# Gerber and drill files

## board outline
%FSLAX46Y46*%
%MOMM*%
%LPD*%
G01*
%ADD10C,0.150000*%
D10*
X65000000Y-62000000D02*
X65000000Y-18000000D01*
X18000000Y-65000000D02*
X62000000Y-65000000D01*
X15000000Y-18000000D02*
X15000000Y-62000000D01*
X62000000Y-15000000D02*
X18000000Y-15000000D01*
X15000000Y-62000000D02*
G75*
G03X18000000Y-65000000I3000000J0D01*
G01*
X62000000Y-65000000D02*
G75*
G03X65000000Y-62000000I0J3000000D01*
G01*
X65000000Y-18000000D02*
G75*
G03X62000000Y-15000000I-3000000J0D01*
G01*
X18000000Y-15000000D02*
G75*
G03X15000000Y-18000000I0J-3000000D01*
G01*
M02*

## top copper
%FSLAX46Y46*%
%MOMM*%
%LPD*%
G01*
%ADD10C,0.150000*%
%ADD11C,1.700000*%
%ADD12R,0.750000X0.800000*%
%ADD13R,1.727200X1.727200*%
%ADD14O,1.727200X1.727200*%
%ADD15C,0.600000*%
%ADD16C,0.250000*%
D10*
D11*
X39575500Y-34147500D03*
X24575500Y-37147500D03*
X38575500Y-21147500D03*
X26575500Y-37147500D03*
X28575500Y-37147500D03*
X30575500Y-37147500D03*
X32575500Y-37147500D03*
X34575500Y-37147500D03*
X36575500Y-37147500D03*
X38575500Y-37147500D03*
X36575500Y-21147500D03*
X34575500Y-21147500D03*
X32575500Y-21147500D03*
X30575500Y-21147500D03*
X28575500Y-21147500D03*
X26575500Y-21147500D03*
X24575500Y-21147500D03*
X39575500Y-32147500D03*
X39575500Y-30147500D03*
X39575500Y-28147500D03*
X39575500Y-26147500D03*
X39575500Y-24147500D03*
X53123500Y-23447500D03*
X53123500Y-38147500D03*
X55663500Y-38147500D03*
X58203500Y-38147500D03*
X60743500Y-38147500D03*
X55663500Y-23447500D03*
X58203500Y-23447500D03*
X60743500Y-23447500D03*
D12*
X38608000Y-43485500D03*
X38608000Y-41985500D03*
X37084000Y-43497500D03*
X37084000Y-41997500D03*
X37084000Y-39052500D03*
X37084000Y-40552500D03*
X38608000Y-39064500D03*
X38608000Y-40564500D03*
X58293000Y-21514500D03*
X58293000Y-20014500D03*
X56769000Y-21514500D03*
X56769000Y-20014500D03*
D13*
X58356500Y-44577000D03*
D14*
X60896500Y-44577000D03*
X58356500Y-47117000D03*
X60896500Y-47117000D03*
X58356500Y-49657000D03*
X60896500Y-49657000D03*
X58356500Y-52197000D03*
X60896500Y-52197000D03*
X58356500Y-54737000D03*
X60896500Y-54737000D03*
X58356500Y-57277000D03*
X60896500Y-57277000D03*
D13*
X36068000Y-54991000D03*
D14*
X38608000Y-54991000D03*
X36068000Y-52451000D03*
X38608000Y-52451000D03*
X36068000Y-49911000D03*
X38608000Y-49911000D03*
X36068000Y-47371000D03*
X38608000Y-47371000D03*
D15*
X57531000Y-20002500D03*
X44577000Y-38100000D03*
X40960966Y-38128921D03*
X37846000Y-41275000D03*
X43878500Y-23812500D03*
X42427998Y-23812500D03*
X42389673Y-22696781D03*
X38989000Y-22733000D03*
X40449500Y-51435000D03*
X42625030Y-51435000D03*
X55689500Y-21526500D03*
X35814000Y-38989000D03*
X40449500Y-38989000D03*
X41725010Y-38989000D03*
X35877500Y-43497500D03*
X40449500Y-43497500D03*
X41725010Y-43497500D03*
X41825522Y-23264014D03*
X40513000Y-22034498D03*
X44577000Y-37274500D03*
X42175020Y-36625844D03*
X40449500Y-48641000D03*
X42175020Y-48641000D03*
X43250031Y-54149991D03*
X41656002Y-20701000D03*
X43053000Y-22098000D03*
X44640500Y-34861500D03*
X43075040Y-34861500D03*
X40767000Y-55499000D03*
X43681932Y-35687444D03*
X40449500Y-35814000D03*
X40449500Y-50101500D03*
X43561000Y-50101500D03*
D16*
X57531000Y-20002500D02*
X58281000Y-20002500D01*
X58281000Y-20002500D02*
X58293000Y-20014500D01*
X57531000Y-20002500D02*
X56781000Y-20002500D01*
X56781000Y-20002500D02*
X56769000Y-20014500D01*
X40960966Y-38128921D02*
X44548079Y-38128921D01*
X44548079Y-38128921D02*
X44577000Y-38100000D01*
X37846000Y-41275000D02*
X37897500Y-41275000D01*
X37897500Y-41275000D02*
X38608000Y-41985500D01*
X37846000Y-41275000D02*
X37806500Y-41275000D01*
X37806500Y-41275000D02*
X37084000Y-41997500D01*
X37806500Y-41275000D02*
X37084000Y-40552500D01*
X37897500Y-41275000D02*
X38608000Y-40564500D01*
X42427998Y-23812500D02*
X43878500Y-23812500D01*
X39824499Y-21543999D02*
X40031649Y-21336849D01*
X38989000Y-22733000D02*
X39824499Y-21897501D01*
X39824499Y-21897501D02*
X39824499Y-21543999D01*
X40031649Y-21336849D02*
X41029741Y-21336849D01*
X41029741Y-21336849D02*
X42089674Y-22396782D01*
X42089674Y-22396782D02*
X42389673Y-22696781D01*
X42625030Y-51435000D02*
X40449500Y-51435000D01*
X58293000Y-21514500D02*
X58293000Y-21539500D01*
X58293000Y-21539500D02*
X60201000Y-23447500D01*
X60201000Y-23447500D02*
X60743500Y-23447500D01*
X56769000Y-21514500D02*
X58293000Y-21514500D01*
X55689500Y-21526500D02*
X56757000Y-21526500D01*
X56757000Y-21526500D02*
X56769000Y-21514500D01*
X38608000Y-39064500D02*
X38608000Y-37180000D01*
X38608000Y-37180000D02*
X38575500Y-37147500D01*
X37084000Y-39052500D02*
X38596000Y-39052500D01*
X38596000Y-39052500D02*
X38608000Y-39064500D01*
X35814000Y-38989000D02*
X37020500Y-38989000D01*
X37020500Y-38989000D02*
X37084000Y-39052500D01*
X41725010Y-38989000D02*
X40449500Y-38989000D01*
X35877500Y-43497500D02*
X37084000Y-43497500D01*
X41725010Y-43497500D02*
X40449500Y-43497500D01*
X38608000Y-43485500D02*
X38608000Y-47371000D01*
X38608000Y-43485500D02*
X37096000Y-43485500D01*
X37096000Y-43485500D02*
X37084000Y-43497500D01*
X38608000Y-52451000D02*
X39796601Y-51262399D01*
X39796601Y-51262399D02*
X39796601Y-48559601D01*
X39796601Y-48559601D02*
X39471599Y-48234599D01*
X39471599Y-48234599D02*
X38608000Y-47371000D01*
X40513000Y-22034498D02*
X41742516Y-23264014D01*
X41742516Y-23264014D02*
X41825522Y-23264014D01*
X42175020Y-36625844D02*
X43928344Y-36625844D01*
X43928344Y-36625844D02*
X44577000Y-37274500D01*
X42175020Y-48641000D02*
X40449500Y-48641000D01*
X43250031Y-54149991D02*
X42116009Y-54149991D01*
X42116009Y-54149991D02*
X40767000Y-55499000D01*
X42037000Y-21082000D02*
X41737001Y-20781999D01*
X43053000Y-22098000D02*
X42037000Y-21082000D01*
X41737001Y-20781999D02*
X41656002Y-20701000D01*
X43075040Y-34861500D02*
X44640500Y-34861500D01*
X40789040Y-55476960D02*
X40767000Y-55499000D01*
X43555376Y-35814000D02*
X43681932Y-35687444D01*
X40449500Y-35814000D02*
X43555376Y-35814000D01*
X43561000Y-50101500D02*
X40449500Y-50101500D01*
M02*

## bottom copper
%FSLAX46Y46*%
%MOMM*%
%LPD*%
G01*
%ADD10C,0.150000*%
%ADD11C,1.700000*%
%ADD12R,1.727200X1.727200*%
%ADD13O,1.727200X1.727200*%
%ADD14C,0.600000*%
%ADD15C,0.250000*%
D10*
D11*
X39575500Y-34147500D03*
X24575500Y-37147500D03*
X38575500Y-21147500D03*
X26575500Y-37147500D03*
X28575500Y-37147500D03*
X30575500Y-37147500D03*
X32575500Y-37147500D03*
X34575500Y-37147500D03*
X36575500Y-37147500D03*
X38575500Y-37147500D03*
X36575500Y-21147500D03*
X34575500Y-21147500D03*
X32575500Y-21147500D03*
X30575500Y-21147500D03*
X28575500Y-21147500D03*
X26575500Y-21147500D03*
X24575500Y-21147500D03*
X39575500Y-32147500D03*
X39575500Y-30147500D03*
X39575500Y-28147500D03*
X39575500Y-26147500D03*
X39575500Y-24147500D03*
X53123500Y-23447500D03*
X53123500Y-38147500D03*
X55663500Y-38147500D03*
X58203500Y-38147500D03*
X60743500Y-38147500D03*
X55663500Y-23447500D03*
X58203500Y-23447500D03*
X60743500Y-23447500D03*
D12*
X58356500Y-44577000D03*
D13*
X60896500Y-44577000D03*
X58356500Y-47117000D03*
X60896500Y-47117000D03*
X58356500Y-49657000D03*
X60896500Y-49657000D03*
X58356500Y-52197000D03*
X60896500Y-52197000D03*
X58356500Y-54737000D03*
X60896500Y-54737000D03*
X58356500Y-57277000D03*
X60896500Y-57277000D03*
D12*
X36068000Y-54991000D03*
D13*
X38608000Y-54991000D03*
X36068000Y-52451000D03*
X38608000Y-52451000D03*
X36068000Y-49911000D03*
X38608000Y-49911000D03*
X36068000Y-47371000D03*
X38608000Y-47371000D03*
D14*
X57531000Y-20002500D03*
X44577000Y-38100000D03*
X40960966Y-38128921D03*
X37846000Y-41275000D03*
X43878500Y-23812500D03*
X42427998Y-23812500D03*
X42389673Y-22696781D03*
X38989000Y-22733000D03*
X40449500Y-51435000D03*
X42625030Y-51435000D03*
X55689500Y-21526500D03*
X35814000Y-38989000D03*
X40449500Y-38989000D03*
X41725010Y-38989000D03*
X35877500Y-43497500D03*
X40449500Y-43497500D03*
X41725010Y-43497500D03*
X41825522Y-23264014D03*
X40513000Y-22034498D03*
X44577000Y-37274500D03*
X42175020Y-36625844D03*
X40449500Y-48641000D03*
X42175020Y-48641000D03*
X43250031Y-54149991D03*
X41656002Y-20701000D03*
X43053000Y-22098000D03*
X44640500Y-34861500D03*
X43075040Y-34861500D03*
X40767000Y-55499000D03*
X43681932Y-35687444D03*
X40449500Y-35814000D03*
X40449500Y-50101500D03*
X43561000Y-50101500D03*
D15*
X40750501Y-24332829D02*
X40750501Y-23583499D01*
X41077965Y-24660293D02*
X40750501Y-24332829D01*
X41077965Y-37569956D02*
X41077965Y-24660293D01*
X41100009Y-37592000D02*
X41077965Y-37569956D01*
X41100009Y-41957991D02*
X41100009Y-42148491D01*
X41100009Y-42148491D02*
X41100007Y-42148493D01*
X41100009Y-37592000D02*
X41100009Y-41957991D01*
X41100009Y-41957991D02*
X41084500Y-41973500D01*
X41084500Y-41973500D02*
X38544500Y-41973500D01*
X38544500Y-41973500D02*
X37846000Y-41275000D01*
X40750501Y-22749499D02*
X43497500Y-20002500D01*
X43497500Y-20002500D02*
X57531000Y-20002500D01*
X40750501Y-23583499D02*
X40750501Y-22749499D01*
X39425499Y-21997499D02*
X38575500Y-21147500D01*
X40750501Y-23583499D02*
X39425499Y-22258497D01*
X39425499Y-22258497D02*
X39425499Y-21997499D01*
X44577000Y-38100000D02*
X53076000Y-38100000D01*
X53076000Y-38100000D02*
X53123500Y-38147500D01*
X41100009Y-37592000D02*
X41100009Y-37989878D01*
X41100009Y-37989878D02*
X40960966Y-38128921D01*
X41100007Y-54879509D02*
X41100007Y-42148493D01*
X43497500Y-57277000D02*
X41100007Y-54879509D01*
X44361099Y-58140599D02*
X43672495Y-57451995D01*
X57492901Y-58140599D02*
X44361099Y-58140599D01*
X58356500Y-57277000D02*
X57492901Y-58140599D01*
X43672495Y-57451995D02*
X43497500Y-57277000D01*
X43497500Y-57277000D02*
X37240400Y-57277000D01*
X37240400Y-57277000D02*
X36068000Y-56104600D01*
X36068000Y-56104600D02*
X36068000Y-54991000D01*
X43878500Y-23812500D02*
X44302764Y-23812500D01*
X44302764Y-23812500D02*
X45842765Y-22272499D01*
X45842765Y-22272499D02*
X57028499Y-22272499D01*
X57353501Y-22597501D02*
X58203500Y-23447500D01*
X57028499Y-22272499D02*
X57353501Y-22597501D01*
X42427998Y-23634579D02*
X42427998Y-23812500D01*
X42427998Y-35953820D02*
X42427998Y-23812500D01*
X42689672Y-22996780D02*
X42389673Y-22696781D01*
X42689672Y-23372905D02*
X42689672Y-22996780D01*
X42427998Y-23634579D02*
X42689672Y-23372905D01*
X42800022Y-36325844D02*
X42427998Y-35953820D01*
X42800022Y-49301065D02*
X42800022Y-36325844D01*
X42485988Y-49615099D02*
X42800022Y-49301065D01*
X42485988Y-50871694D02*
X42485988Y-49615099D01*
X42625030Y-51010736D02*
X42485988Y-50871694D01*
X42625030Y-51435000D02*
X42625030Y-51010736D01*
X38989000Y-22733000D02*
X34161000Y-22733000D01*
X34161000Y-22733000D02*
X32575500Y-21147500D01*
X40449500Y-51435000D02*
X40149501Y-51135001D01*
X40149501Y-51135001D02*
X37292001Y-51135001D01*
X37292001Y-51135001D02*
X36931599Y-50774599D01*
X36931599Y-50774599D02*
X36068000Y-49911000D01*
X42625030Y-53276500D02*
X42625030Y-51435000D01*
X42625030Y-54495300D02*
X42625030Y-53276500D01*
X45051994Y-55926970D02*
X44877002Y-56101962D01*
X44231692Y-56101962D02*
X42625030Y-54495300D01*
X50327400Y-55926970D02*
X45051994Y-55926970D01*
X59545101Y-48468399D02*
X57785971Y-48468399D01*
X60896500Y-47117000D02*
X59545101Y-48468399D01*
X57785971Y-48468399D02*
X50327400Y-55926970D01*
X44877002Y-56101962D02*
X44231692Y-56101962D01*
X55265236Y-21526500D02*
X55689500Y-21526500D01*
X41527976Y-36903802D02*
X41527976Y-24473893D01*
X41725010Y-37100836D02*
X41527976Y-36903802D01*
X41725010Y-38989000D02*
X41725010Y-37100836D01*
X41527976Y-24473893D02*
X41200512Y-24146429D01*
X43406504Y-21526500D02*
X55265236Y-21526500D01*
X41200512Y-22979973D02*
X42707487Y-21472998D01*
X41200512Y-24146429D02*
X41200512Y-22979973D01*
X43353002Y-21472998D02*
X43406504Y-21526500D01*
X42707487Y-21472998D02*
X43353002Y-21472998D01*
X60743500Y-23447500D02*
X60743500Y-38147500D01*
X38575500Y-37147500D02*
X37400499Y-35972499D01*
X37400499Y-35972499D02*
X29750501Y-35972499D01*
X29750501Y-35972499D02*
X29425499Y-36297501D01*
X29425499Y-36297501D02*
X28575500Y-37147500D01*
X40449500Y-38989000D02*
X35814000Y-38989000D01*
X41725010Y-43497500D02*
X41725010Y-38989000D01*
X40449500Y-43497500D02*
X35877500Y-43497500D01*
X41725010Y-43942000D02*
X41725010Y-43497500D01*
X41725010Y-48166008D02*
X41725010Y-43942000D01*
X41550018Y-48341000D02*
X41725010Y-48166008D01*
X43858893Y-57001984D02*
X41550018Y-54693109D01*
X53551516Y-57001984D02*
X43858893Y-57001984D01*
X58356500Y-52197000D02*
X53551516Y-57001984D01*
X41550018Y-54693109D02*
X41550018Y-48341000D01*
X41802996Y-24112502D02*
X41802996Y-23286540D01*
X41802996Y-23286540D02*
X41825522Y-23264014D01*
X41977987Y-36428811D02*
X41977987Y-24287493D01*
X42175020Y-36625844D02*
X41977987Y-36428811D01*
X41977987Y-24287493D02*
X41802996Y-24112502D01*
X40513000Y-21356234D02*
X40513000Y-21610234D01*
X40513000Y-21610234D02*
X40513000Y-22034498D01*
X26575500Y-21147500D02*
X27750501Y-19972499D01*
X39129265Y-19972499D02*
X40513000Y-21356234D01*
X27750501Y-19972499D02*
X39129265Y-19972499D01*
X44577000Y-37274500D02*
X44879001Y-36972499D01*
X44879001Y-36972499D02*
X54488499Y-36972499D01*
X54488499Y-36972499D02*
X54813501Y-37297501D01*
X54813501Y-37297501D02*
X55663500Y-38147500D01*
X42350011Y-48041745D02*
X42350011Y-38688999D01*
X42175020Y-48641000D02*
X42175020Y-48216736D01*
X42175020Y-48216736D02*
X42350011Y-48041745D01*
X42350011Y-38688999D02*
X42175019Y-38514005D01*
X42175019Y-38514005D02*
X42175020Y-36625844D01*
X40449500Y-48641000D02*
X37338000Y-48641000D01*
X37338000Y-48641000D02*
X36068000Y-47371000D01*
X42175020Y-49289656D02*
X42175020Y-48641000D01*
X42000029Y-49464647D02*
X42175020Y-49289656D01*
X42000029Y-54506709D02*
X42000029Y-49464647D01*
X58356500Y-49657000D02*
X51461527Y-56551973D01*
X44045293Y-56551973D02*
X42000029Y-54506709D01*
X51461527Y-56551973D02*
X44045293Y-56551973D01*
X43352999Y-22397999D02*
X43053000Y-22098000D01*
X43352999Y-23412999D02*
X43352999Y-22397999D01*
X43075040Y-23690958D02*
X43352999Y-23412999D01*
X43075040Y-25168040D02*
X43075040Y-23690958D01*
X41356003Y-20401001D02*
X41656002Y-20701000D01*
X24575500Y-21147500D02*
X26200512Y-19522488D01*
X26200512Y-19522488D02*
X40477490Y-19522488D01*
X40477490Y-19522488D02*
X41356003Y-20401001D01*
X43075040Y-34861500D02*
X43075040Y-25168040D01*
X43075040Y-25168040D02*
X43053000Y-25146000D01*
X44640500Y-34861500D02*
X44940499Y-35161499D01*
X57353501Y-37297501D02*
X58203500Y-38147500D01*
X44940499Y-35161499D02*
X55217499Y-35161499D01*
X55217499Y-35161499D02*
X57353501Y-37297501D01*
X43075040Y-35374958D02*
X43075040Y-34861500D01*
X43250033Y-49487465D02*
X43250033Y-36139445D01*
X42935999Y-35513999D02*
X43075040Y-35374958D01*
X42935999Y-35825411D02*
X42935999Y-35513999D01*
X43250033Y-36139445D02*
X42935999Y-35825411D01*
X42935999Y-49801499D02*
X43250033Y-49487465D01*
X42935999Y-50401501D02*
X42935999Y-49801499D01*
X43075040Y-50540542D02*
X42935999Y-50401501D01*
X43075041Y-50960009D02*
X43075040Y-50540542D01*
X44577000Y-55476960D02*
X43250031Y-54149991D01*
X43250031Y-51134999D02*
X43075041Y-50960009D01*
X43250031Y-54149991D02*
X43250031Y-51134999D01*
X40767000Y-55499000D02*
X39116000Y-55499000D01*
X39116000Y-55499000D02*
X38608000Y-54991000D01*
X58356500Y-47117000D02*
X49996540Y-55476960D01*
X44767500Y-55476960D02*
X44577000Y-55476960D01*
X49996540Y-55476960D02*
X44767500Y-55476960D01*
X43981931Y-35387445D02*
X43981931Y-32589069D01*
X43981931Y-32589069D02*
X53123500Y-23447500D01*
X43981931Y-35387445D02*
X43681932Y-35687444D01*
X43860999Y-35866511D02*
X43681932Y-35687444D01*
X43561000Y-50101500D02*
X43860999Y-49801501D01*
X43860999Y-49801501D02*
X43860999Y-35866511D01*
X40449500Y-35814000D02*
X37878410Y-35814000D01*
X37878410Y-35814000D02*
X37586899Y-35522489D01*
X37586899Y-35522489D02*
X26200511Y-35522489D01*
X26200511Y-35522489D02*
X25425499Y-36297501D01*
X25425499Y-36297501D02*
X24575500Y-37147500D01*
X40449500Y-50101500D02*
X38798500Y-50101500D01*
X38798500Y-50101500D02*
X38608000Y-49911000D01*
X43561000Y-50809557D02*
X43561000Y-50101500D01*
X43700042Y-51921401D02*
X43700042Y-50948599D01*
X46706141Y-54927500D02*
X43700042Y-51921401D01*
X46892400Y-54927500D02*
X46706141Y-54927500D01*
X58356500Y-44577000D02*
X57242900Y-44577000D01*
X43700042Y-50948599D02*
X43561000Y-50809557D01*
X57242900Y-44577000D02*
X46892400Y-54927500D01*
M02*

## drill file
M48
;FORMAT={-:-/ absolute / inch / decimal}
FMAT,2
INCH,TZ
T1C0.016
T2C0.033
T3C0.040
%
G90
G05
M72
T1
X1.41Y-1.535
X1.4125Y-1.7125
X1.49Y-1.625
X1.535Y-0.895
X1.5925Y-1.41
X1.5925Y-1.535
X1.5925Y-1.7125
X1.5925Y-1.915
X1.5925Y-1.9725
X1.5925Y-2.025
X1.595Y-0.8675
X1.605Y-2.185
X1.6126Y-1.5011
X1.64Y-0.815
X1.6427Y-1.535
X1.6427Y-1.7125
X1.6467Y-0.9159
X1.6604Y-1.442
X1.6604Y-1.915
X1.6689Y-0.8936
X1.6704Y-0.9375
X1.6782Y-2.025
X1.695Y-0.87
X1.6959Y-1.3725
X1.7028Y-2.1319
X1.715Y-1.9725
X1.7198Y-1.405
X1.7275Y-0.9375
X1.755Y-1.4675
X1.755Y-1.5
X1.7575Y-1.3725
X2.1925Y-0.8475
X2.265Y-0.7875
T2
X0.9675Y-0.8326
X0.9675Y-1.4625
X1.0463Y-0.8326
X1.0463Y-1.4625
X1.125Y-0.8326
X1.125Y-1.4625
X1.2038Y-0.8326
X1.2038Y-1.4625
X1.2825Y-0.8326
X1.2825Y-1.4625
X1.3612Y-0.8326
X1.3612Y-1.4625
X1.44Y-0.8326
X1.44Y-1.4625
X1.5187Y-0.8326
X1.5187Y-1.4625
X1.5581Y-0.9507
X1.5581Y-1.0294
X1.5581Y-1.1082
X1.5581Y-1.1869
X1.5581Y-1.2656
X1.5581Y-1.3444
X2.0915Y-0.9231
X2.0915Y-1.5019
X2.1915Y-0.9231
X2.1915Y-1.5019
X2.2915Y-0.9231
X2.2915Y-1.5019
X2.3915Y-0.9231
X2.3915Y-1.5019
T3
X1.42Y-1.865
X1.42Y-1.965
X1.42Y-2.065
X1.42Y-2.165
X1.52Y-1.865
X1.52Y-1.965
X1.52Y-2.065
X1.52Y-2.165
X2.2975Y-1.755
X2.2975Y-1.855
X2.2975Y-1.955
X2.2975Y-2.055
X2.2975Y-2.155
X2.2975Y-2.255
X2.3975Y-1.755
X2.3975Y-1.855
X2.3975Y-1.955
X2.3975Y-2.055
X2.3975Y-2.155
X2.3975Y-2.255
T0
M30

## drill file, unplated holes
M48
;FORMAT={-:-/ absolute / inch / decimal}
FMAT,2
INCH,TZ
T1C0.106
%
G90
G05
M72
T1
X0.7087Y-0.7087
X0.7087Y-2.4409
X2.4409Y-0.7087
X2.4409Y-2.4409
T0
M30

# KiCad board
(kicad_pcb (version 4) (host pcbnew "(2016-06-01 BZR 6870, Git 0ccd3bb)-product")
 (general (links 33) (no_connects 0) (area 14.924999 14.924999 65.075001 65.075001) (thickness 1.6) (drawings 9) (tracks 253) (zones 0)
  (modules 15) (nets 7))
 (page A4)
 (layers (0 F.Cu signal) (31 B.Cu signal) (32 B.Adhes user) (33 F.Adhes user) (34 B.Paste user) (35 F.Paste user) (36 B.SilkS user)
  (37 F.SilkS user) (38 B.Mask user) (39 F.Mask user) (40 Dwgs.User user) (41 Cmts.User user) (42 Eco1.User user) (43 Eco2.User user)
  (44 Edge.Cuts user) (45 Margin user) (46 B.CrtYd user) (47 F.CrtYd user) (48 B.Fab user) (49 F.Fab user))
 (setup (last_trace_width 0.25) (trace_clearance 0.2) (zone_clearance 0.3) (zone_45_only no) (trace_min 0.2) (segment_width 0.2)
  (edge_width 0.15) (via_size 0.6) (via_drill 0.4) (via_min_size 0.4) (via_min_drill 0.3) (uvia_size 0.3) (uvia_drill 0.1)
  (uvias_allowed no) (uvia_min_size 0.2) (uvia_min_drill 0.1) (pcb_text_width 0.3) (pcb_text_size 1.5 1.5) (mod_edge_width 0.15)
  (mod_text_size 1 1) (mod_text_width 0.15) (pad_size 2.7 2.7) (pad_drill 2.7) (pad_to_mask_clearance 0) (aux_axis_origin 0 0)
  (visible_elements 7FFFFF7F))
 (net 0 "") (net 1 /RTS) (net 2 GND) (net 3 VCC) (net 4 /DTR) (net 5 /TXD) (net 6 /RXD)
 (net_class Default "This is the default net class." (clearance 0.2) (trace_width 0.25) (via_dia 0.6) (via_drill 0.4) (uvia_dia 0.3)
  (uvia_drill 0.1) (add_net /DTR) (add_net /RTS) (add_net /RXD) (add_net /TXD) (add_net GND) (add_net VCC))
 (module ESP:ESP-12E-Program (layer F.Cu) (at 27.5755 29.1475 90)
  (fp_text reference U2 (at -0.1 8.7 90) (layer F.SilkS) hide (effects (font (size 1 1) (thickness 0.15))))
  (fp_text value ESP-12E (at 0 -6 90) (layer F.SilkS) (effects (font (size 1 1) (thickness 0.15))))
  (pad 9 thru_hole circle (at -5 12 90) (size 1.7 1.7) (drill 0.85) (layers *.Cu *.Mask F.SilkS))
  (pad 1 thru_hole circle (at -8 -3 90) (size 1.7 1.7) (drill 0.85) (layers *.Cu *.Mask F.SilkS) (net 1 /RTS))
  (pad 15 thru_hole circle (at 8 11 90) (size 1.7 1.7) (drill 0.85) (layers *.Cu *.Mask F.SilkS) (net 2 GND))
  (pad 2 thru_hole circle (at -8 -1 90) (size 1.7 1.7) (drill 0.85) (layers *.Cu *.Mask F.SilkS))
  (pad 3 thru_hole circle (at -8 1 90) (size 1.7 1.7) (drill 0.85) (layers *.Cu *.Mask F.SilkS) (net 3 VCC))
  (pad 4 thru_hole circle (at -8 3 90) (size 1.7 1.7) (drill 0.85) (layers *.Cu *.Mask F.SilkS))
  (pad 5 thru_hole circle (at -8 5 90) (size 1.7 1.7) (drill 0.85) (layers *.Cu *.Mask F.SilkS))
  (pad 6 thru_hole circle (at -8 7 90) (size 1.7 1.7) (drill 0.85) (layers *.Cu *.Mask F.SilkS))
  (pad 7 thru_hole circle (at -8 9 90) (size 1.7 1.7) (drill 0.85) (layers *.Cu *.Mask F.SilkS))
  (pad 8 thru_hole circle (at -8 11 90) (size 1.7 1.7) (drill 0.85) (layers *.Cu *.Mask F.SilkS) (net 3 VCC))
  (pad 16 thru_hole circle (at 8 9 90) (size 1.7 1.7) (drill 0.85) (layers *.Cu *.Mask F.SilkS))
  (pad 17 thru_hole circle (at 8 7 90) (size 1.7 1.7) (drill 0.85) (layers *.Cu *.Mask F.SilkS))
  (pad 18 thru_hole circle (at 8 5 90) (size 1.7 1.7) (drill 0.85) (layers *.Cu *.Mask F.SilkS) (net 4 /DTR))
  (pad 19 thru_hole circle (at 8 3 90) (size 1.7 1.7) (drill 0.85) (layers *.Cu *.Mask F.SilkS))
  (pad 20 thru_hole circle (at 8 1 90) (size 1.7 1.7) (drill 0.85) (layers *.Cu *.Mask F.SilkS))
  (pad 21 thru_hole circle (at 8 -1 90) (size 1.7 1.7) (drill 0.85) (layers *.Cu *.Mask F.SilkS) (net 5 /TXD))
  (pad 22 thru_hole circle (at 8 -3 90) (size 1.7 1.7) (drill 0.85) (layers *.Cu *.Mask F.SilkS) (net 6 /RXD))
  (pad 10 thru_hole circle (at -3 12 90) (size 1.7 1.7) (drill 0.85) (layers *.Cu *.Mask F.SilkS))
  (pad 11 thru_hole circle (at -1 12 90) (size 1.7 1.7) (drill 0.85) (layers *.Cu *.Mask F.SilkS))
  (pad 12 thru_hole circle (at 1 12 90) (size 1.7 1.7) (drill 0.85) (layers *.Cu *.Mask F.SilkS))
  (pad 13 thru_hole circle (at 3 12 90) (size 1.7 1.7) (drill 0.85) (layers *.Cu *.Mask F.SilkS))
  (pad 14 thru_hole circle (at 5 12 90) (size 1.7 1.7) (drill 0.85) (layers *.Cu *.Mask F.SilkS)))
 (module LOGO (layer F.Cu) (at 49.022 53.467 90)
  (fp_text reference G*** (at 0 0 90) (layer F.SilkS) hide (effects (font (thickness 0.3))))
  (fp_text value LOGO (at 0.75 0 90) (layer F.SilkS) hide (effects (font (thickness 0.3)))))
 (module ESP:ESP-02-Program (layer F.Cu) (at 54.6735 30.7975 90)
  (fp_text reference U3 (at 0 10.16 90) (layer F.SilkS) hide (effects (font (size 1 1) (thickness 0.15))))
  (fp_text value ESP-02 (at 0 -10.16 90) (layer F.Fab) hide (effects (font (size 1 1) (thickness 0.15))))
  (pad 8 thru_hole circle (at 7.35 -1.55 90) (size 1.7 1.7) (drill 0.85) (layers *.Cu *.Mask F.SilkS) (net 1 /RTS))
  (pad 1 thru_hole circle (at -7.35 -1.55 90) (size 1.7 1.7) (drill 0.85) (layers *.Cu *.Mask F.SilkS) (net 2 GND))
  (pad 2 thru_hole circle (at -7.35 0.99 90) (size 1.7 1.7) (drill 0.85) (layers *.Cu *.Mask F.SilkS) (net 5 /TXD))
  (pad 3 thru_hole circle (at -7.35 3.53 90) (size 1.7 1.7) (drill 0.85) (layers *.Cu *.Mask F.SilkS) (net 6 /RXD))
  (pad 4 thru_hole circle (at -7.35 6.07 90) (size 1.7 1.7) (drill 0.85) (layers *.Cu *.Mask F.SilkS) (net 3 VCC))
  (pad 7 thru_hole circle (at 7.35 0.99 90) (size 1.7 1.7) (drill 0.85) (layers *.Cu *.Mask F.SilkS))
  (pad 6 thru_hole circle (at 7.35 3.53 90) (size 1.7 1.7) (drill 0.85) (layers *.Cu *.Mask F.SilkS) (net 4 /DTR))
  (pad 5 thru_hole circle (at 7.35 6.07 90) (size 1.7 1.7) (drill 0.85) (layers *.Cu *.Mask F.SilkS) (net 3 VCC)))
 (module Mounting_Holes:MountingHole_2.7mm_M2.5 (layer F.Cu) (at 18 18)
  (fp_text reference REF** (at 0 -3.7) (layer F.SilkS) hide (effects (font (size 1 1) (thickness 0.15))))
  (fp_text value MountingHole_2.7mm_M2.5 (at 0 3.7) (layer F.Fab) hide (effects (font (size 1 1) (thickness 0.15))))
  (pad "" np_thru_hole circle (at 0 0) (size 2.7 2.7) (drill 2.7) (layers *.Cu *.Mask F.SilkS)))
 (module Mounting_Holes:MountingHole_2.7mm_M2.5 (layer F.Cu) (at 18 62)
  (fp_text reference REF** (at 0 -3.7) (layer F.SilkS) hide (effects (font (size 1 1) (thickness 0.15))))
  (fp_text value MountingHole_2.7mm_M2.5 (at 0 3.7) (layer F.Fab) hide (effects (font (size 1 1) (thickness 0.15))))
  (pad 1 np_thru_hole circle (at 0 0) (size 2.7 2.7) (drill 2.7) (layers *.Cu *.Mask F.SilkS)))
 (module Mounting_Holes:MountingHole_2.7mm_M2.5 (layer F.Cu) (at 62 62)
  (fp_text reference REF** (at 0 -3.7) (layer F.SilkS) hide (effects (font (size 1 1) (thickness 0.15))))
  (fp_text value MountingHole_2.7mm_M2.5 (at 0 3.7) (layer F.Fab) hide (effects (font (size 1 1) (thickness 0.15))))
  (pad 1 np_thru_hole circle (at 0 0) (size 2.7 2.7) (drill 2.7) (layers *.Cu *.Mask F.SilkS)))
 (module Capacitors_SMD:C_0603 (layer F.Cu) (at 38.608 42.7355 90)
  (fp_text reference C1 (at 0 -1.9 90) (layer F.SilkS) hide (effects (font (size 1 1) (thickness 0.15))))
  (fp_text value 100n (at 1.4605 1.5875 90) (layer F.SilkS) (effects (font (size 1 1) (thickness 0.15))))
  (pad 1 smd rect (at -0.75 0 90) (size 0.8 0.75) (layers F.Cu F.Paste F.Mask) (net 3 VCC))
  (pad 2 smd rect (at 0.75 0 90) (size 0.8 0.75) (layers F.Cu F.Paste F.Mask) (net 2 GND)))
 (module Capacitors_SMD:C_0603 (layer F.Cu) (at 37.084 42.7475 90)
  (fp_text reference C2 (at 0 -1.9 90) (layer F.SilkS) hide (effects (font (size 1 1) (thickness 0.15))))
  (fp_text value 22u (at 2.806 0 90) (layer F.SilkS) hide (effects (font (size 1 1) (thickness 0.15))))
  (pad 1 smd rect (at -0.75 0 90) (size 0.8 0.75) (layers F.Cu F.Paste F.Mask) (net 3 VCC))
  (pad 2 smd rect (at 0.75 0 90) (size 0.8 0.75) (layers F.Cu F.Paste F.Mask) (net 2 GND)))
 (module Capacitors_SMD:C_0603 (layer F.Cu) (at 37.084 39.8025 270)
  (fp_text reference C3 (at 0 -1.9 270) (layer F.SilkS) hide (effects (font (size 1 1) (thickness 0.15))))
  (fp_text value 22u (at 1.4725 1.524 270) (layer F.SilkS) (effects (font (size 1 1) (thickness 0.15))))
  (pad 1 smd rect (at -0.75 0 270) (size 0.8 0.75) (layers F.Cu F.Paste F.Mask) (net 3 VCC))
  (pad 2 smd rect (at 0.75 0 270) (size 0.8 0.75) (layers F.Cu F.Paste F.Mask) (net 2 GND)))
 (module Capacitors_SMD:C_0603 (layer F.Cu) (at 38.608 39.8145 270)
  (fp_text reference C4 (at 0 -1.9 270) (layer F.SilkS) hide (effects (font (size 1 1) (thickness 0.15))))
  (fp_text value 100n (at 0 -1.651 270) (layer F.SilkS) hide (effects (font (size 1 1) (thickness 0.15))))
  (pad 1 smd rect (at -0.75 0 270) (size 0.8 0.75) (layers F.Cu F.Paste F.Mask) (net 3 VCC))
  (pad 2 smd rect (at 0.75 0 270) (size 0.8 0.75) (layers F.Cu F.Paste F.Mask) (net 2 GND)))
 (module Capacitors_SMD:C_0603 (layer F.Cu) (at 58.293 20.7645 90)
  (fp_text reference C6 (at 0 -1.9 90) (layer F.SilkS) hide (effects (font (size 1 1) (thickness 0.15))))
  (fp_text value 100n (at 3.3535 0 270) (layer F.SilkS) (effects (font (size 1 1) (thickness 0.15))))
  (pad 1 smd rect (at -0.75 0 90) (size 0.8 0.75) (layers F.Cu F.Paste F.Mask) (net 3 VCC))
  (pad 2 smd rect (at 0.75 0 90) (size 0.8 0.75) (layers F.Cu F.Paste F.Mask) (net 2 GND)))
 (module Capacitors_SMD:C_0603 (layer F.Cu) (at 56.769 20.7645 90)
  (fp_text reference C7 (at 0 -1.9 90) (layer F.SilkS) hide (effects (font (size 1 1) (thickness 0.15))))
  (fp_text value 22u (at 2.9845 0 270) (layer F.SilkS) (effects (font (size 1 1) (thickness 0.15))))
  (pad 1 smd rect (at -0.75 0 90) (size 0.8 0.75) (layers F.Cu F.Paste F.Mask) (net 3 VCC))
  (pad 2 smd rect (at 0.75 0 90) (size 0.8 0.75) (layers F.Cu F.Paste F.Mask) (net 2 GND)))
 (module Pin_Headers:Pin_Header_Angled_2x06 (layer F.Cu) (at 58.3565 44.577)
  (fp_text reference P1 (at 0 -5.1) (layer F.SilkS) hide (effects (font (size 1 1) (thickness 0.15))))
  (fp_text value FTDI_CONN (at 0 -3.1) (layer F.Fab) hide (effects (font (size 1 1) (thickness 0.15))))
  (pad 1 thru_hole rect (at 0 0) (size 1.7272 1.7272) (drill 1.016) (layers *.Cu *.Mask F.SilkS) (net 1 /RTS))
  (pad 2 thru_hole oval (at 2.54 0) (size 1.7272 1.7272) (drill 1.016) (layers *.Cu *.Mask F.SilkS))
  (pad 3 thru_hole oval (at 0 2.54) (size 1.7272 1.7272) (drill 1.016) (layers *.Cu *.Mask F.SilkS) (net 6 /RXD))
  (pad 4 thru_hole oval (at 2.54 2.54) (size 1.7272 1.7272) (drill 1.016) (layers *.Cu *.Mask F.SilkS) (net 4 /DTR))
  (pad 5 thru_hole oval (at 0 5.08) (size 1.7272 1.7272) (drill 1.016) (layers *.Cu *.Mask F.SilkS) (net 5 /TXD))
  (pad 6 thru_hole oval (at 2.54 5.08) (size 1.7272 1.7272) (drill 1.016) (layers *.Cu *.Mask F.SilkS))
  (pad 7 thru_hole oval (at 0 7.62) (size 1.7272 1.7272) (drill 1.016) (layers *.Cu *.Mask F.SilkS) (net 3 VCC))
  (pad 8 thru_hole oval (at 2.54 7.62) (size 1.7272 1.7272) (drill 1.016) (layers *.Cu *.Mask F.SilkS))
  (pad 9 thru_hole oval (at 0 10.16) (size 1.7272 1.7272) (drill 1.016) (layers *.Cu *.Mask F.SilkS))
  (pad 10 thru_hole oval (at 2.54 10.16) (size 1.7272 1.7272) (drill 1.016) (layers *.Cu *.Mask F.SilkS))
  (pad 11 thru_hole oval (at 0 12.7) (size 1.7272 1.7272) (drill 1.016) (layers *.Cu *.Mask F.SilkS) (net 2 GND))
  (pad 12 thru_hole oval (at 2.54 12.7) (size 1.7272 1.7272) (drill 1.016) (layers *.Cu *.Mask F.SilkS)))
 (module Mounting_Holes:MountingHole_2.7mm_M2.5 (layer F.Cu) (at 62 18)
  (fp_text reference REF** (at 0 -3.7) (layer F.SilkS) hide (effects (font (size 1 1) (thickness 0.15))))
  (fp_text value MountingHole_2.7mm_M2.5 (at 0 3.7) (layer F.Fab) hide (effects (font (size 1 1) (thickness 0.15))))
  (pad 1 np_thru_hole circle (at 0 0) (size 2.7 2.7) (drill 2.7) (layers *.Cu *.Mask F.SilkS)))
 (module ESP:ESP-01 (layer F.Cu) (at 37.338 51.181 90)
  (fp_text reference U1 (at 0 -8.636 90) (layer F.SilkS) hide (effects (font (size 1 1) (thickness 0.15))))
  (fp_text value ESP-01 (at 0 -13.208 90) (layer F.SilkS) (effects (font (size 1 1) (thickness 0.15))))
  (pad 1 thru_hole rect (at -3.81 -1.27 90) (size 1.7272 1.7272) (drill 1.016) (layers *.Cu *.Mask F.SilkS) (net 2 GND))
  (pad 2 thru_hole oval (at -3.81 1.27 90) (size 1.7272 1.7272) (drill 1.016) (layers *.Cu *.Mask F.SilkS) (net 6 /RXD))
  (pad 3 thru_hole oval (at -1.27 -1.27 90) (size 1.7272 1.7272) (drill 1.016) (layers *.Cu *.Mask F.SilkS))
  (pad 4 thru_hole oval (at -1.27 1.27 90) (size 1.7272 1.7272) (drill 1.016) (layers *.Cu *.Mask F.SilkS) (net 3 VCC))
  (pad 5 thru_hole oval (at 1.27 -1.27 90) (size 1.7272 1.7272) (drill 1.016) (layers *.Cu *.Mask F.SilkS) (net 4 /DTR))
  (pad 6 thru_hole oval (at 1.27 1.27 90) (size 1.7272 1.7272) (drill 1.016) (layers *.Cu *.Mask F.SilkS) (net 1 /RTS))
  (pad 7 thru_hole oval (at 3.81 -1.27 90) (size 1.7272 1.7272) (drill 1.016) (layers *.Cu *.Mask F.SilkS) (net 5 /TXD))
  (pad 8 thru_hole oval (at 3.81 1.27 90) (size 1.7272 1.7272) (drill 1.016) (layers *.Cu *.Mask F.SilkS) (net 3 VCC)))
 (gr_line (start 65 62) (end 65 18) (layer Edge.Cuts) (width 0.15))
 (gr_line (start 18 65) (end 62 65) (layer Edge.Cuts) (width 0.15))
 (gr_line (start 15 18) (end 15 62) (layer Edge.Cuts) (width 0.15))
 (gr_line (start 62 15) (end 18 15) (layer Edge.Cuts) (width 0.15))
 (gr_arc (start 18 62) (end 18 65) (angle 90) (layer Edge.Cuts) (width 0.15))
 (gr_arc (start 62 62) (end 65 62) (angle 90) (layer Edge.Cuts) (width 0.15))
 (gr_arc (start 62 18) (end 62 15) (angle 90) (layer Edge.Cuts) (width 0.15))
 (gr_arc (start 18 18) (end 15 18) (angle 90) (layer Edge.Cuts) (width 0.15))
 (segment (start 40.750501 24.332829) (end 40.750501 23.583499) (width 0.25) (layer B.Cu) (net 2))
 (segment (start 41.077965 24.660293) (end 40.750501 24.332829) (width 0.25) (layer B.Cu) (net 2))
 (segment (start 41.077965 37.569956) (end 41.077965 24.660293) (width 0.25) (layer B.Cu) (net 2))
 (segment (start 41.100009 37.592) (end 41.077965 37.569956) (width 0.25) (layer B.Cu) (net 2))
 (segment (start 41.100009 41.957991) (end 41.100009 42.148491) (width 0.25) (layer B.Cu) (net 2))
 (segment (start 41.100009 42.148491) (end 41.100007 42.148493) (width 0.25) (layer B.Cu) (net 2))
 (segment (start 41.100009 37.592) (end 41.100009 41.957991) (width 0.25) (layer B.Cu) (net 2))
 (segment (start 41.100009 41.957991) (end 41.0845 41.9735) (width 0.25) (layer B.Cu) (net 2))
 (segment (start 41.0845 41.9735) (end 38.5445 41.9735) (width 0.25) (layer B.Cu) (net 2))
 (segment (start 38.5445 41.9735) (end 37.846 41.275) (width 0.25) (layer B.Cu) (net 2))
 (segment (start 57.531 20.0025) (end 58.281 20.0025) (width 0.25) (layer F.Cu) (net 2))
 (segment (start 58.281 20.0025) (end 58.293 20.0145) (width 0.25) (layer F.Cu) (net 2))
 (segment (start 57.531 20.0025) (end 56.781 20.0025) (width 0.25) (layer F.Cu) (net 2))
 (segment (start 56.781 20.0025) (end 56.769 20.0145) (width 0.25) (layer F.Cu) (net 2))
 (segment (start 40.750501 22.749499) (end 43.4975 20.0025) (width 0.25) (layer B.Cu) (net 2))
 (segment (start 43.4975 20.0025) (end 57.531 20.0025) (width 0.25) (layer B.Cu) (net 2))
 (via (at 57.531 20.0025) (size 0.6) (drill 0.4) (layers F.Cu B.Cu) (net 2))
 (segment (start 40.750501 23.583499) (end 40.750501 22.749499) (width 0.25) (layer B.Cu) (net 2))
 (segment (start 39.425499 21.997499) (end 38.5755 21.1475) (width 0.25) (layer B.Cu) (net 2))
 (segment (start 40.750501 23.583499) (end 39.425499 22.258497) (width 0.25) (layer B.Cu) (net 2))
 (segment (start 39.425499 22.258497) (end 39.425499 21.997499) (width 0.25) (layer B.Cu) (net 2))
 (segment (start 44.577 38.1) (end 53.076 38.1) (width 0.25) (layer B.Cu) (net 2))
 (segment (start 53.076 38.1) (end 53.1235 38.1475) (width 0.25) (layer B.Cu) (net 2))
 (segment (start 40.960966 38.128921) (end 44.548079 38.128921) (width 0.25) (layer F.Cu) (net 2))
 (segment (start 44.548079 38.128921) (end 44.577 38.1) (width 0.25) (layer F.Cu) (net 2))
 (via (at 44.577 38.1) (size 0.6) (drill 0.4) (layers F.Cu B.Cu) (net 2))
 (segment (start 41.100009 37.592) (end 41.100009 37.989878) (width 0.25) (layer B.Cu) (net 2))
 (segment (start 41.100009 37.989878) (end 40.960966 38.128921) (width 0.25) (layer B.Cu) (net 2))
 (via (at 40.960966 38.128921) (size 0.6) (drill 0.4) (layers F.Cu B.Cu) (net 2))
 (segment (start 41.100007 54.879509) (end 41.100007 42.148493) (width 0.25) (layer B.Cu) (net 2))
 (segment (start 43.4975 57.277) (end 41.100007 54.879509) (width 0.25) (layer B.Cu) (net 2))
 (segment (start 37.846 41.275) (end 37.8975 41.275) (width 0.25) (layer F.Cu) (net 2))
 (segment (start 37.8975 41.275) (end 38.608 41.9855) (width 0.25) (layer F.Cu) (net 2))
 (segment (start 37.846 41.275) (end 37.8065 41.275) (width 0.25) (layer F.Cu) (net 2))
 (segment (start 37.8065 41.275) (end 37.084 41.9975) (width 0.25) (layer F.Cu) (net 2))
 (segment (start 37.8065 41.275) (end 37.084 40.5525) (width 0.25) (layer F.Cu) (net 2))
 (segment (start 37.8975 41.275) (end 38.608 40.5645) (width 0.25) (layer F.Cu) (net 2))
 (via (at 37.846 41.275) (size 0.6) (drill 0.4) (layers F.Cu B.Cu) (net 2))
 (segment (start 44.361099 58.140599) (end 43.672495 57.451995) (width 0.25) (layer B.Cu) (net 2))
 (segment (start 57.492901 58.140599) (end 44.361099 58.140599) (width 0.25) (layer B.Cu) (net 2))
 (segment (start 58.3565 57.277) (end 57.492901 58.140599) (width 0.25) (layer B.Cu) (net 2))
 (segment (start 43.672495 57.451995) (end 43.4975 57.277) (width 0.25) (layer B.Cu) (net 2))
 (segment (start 43.4975 57.277) (end 37.2404 57.277) (width 0.25) (layer B.Cu) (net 2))
 (segment (start 37.2404 57.277) (end 36.068 56.1046) (width 0.25) (layer B.Cu) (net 2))
 (segment (start 36.068 56.1046) (end 36.068 54.991) (width 0.25) (layer B.Cu) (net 2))
 (segment (start 43.8785 23.8125) (end 44.302764 23.8125) (width 0.25) (layer B.Cu) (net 4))
 (segment (start 44.302764 23.8125) (end 45.842765 22.272499) (width 0.25) (layer B.Cu) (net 4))
 (segment (start 45.842765 22.272499) (end 57.028499 22.272499) (width 0.25) (layer B.Cu) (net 4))
 (segment (start 57.353501 22.597501) (end 58.2035 23.4475) (width 0.25) (layer B.Cu) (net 4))
 (segment (start 57.028499 22.272499) (end 57.353501 22.597501) (width 0.25) (layer B.Cu) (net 4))
 (segment (start 42.427998 23.8125) (end 43.8785 23.8125) (width 0.25) (layer F.Cu) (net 4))
 (via (at 43.8785 23.8125) (size 0.6) (drill 0.4) (layers F.Cu B.Cu) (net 4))
 (via (at 42.427998 23.8125) (size 0.6) (drill 0.4) (layers F.Cu B.Cu) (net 4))
 (segment (start 42.427998 23.634579) (end 42.427998 23.8125) (width 0.25) (layer B.Cu) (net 4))
 (segment (start 42.427998 35.95382) (end 42.427998 23.8125) (width 0.25) (layer B.Cu) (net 4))
 (segment (start 39.824499 21.543999) (end 40.031649 21.336849) (width 0.25) (layer F.Cu) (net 4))
 (segment (start 42.689672 22.99678) (end 42.389673 22.696781) (width 0.25) (layer B.Cu) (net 4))
 (via (at 42.389673 22.696781) (size 0.6) (drill 0.4) (layers F.Cu B.Cu) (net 4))
 (segment (start 42.689672 23.372905) (end 42.689672 22.99678) (width 0.25) (layer B.Cu) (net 4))
 (segment (start 42.427998 23.634579) (end 42.689672 23.372905) (width 0.25) (layer B.Cu) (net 4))
 (segment (start 38.989 22.733) (end 39.824499 21.897501) (width 0.25) (layer F.Cu) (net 4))
 (segment (start 39.824499 21.897501) (end 39.824499 21.543999) (width 0.25) (layer F.Cu) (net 4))
 (segment (start 40.031649 21.336849) (end 41.029741 21.336849) (width 0.25) (layer F.Cu) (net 4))
 (segment (start 41.029741 21.336849) (end 42.089674 22.396782) (width 0.25) (layer F.Cu) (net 4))
 (segment (start 42.089674 22.396782) (end 42.389673 22.696781) (width 0.25) (layer F.Cu) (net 4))
 (segment (start 42.800022 36.325844) (end 42.427998 35.95382) (width 0.25) (layer B.Cu) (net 4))
 (segment (start 42.800022 49.301065) (end 42.800022 36.325844) (width 0.25) (layer B.Cu) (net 4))
 (segment (start 42.485988 49.615099) (end 42.800022 49.301065) (width 0.25) (layer B.Cu) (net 4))
 (segment (start 42.485988 50.871694) (end 42.485988 49.615099) (width 0.25) (layer B.Cu) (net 4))
 (segment (start 42.62503 51.010736) (end 42.485988 50.871694) (width 0.25) (layer B.Cu) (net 4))
 (segment (start 42.62503 51.435) (end 42.62503 51.010736) (width 0.25) (layer B.Cu) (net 4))
 (segment (start 38.989 22.733) (end 34.161 22.733) (width 0.25) (layer B.Cu) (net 4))
 (segment (start 34.161 22.733) (end 32.5755 21.1475) (width 0.25) (layer B.Cu) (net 4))
 (via (at 38.989 22.733) (size 0.6) (drill 0.4) (layers F.Cu B.Cu) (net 4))
 (segment (start 40.4495 51.435) (end 40.149501 51.135001) (width 0.25) (layer B.Cu) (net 4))
 (segment (start 40.149501 51.135001) (end 37.292001 51.135001) (width 0.25) (layer B.Cu) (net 4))
 (segment (start 37.292001 51.135001) (end 36.931599 50.774599) (width 0.25) (layer B.Cu) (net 4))
 (segment (start 36.931599 50.774599) (end 36.068 49.911) (width 0.25) (layer B.Cu) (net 4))
 (segment (start 42.62503 51.435) (end 40.4495 51.435) (width 0.25) (layer F.Cu) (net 4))
 (via (at 40.4495 51.435) (size 0.6) (drill 0.4) (layers F.Cu B.Cu) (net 4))
 (via (at 42.62503 51.435) (size 0.6) (drill 0.4) (layers F.Cu B.Cu) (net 4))
 (segment (start 42.62503 53.2765) (end 42.62503 51.435) (width 0.25) (layer B.Cu) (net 4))
 (segment (start 42.62503 54.4953) (end 42.62503 53.2765) (width 0.25) (layer B.Cu) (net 4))
 (segment (start 45.051994 55.92697) (end 44.877002 56.101962) (width 0.25) (layer B.Cu) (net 4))
 (segment (start 44.231692 56.101962) (end 42.62503 54.4953) (width 0.25) (layer B.Cu) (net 4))
 (segment (start 50.3274 55.92697) (end 45.051994 55.92697) (width 0.25) (layer B.Cu) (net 4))
 (segment (start 59.545101 48.468399) (end 57.785971 48.468399) (width 0.25) (layer B.Cu) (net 4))
 (segment (start 60.8965 47.117) (end 59.545101 48.468399) (width 0.25) (layer B.Cu) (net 4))
 (segment (start 57.785971 48.468399) (end 50.3274 55.92697) (width 0.25) (layer B.Cu) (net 4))
 (segment (start 44.877002 56.101962) (end 44.231692 56.101962) (width 0.25) (layer B.Cu) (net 4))
 (segment (start 55.265236 21.5265) (end 55.6895 21.5265) (width 0.25) (layer B.Cu) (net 3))
 (segment (start 41.527976 36.903802) (end 41.527976 24.473893) (width 0.25) (layer B.Cu) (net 3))
 (segment (start 41.72501 37.100836) (end 41.527976 36.903802) (width 0.25) (layer B.Cu) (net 3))
 (segment (start 41.72501 38.989) (end 41.72501 37.100836) (width 0.25) (layer B.Cu) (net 3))
 (segment (start 41.527976 24.473893) (end 41.200512 24.146429) (width 0.25) (layer B.Cu) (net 3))
 (segment (start 43.406504 21.5265) (end 55.265236 21.5265) (width 0.25) (layer B.Cu) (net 3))
 (segment (start 41.200512 22.979973) (end 42.707487 21.472998) (width 0.25) (layer B.Cu) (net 3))
 (segment (start 41.200512 24.146429) (end 41.200512 22.979973) (width 0.25) (layer B.Cu) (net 3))
 (segment (start 43.353002 21.472998) (end 43.406504 21.5265) (width 0.25) (layer B.Cu) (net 3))
 (segment (start 42.707487 21.472998) (end 43.353002 21.472998) (width 0.25) (layer B.Cu) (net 3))
 (segment (start 60.7435 23.4475) (end 60.7435 38.1475) (width 0.25) (layer B.Cu) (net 3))
 (segment (start 58.293 21.5145) (end 58.293 21.5395) (width 0.25) (layer F.Cu) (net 3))
 (segment (start 58.293 21.5395) (end 60.201 23.4475) (width 0.25) (layer F.Cu) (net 3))
 (segment (start 60.201 23.4475) (end 60.7435 23.4475) (width 0.25) (layer F.Cu) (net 3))
 (segment (start 56.769 21.5145) (end 58.293 21.5145) (width 0.25) (layer F.Cu) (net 3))
 (segment (start 55.6895 21.5265) (end 56.757 21.5265) (width 0.25) (layer F.Cu) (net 3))
 (segment (start 56.757 21.5265) (end 56.769 21.5145) (width 0.25) (layer F.Cu) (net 3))
 (via (at 55.6895 21.5265) (size 0.6) (drill 0.4) (layers F.Cu B.Cu) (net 3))
 (segment (start 38.5755 37.1475) (end 37.400499 35.972499) (width 0.25) (layer B.Cu) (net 3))
 (segment (start 37.400499 35.972499) (end 29.750501 35.972499) (width 0.25) (layer B.Cu) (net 3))
 (segment (start 29.750501 35.972499) (end 29.425499 36.297501) (width 0.25) (layer B.Cu) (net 3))
 (segment (start 29.425499 36.297501) (end 28.5755 37.1475) (width 0.25) (layer B.Cu) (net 3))
 (segment (start 38.608 39.0645) (end 38.608 37.18) (width 0.25) (layer F.Cu) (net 3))
 (segment (start 38.608 37.18) (end 38.5755 37.1475) (width 0.25) (layer F.Cu) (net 3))
 (segment (start 37.084 39.0525) (end 38.596 39.0525) (width 0.25) (layer F.Cu) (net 3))
 (segment (start 38.596 39.0525) (end 38.608 39.0645) (width 0.25) (layer F.Cu) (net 3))
 (segment (start 35.814 38.989) (end 37.0205 38.989) (width 0.25) (layer F.Cu) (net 3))
 (segment (start 37.0205 38.989) (end 37.084 39.0525) (width 0.25) (layer F.Cu) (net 3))
 (segment (start 40.4495 38.989) (end 35.814 38.989) (width 0.25) (layer B.Cu) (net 3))
 (via (at 35.814 38.989) (size 0.6) (drill 0.4) (layers F.Cu B.Cu) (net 3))
 (segment (start 41.72501 38.989) (end 40.4495 38.989) (width 0.25) (layer F.Cu) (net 3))
 (via (at 40.4495 38.989) (size 0.6) (drill 0.4) (layers F.Cu B.Cu) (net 3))
 (segment (start 41.72501 43.4975) (end 41.72501 38.989) (width 0.25) (layer B.Cu) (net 3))
 (via (at 41.72501 38.989) (size 0.6) (drill 0.4) (layers F.Cu B.Cu) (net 3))
 (segment (start 35.8775 43.4975) (end 37.084 43.4975) (width 0.25) (layer F.Cu) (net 3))
 (segment (start 40.4495 43.4975) (end 35.8775 43.4975) (width 0.25) (layer B.Cu) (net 3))
 (via (at 35.8775 43.4975) (size 0.6) (drill 0.4) (layers F.Cu B.Cu) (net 3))
 (segment (start 41.72501 43.4975) (end 40.4495 43.4975) (width 0.25) (layer F.Cu) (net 3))
 (via (at 40.4495 43.4975) (size 0.6) (drill 0.4) (layers F.Cu B.Cu) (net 3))
 (segment (start 38.608 43.4855) (end 38.608 47.371) (width 0.25) (layer F.Cu) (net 3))
 (segment (start 38.608 43.4855) (end 37.096 43.4855) (width 0.25) (layer F.Cu) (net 3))
 (segment (start 37.096 43.4855) (end 37.084 43.4975) (width 0.25) (layer F.Cu) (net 3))
 (segment (start 41.72501 43.942) (end 41.72501 43.4975) (width 0.25) (layer B.Cu) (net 3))
 (via (at 41.72501 43.4975) (size 0.6) (drill 0.4) (layers F.Cu B.Cu) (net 3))
 (segment (start 38.608 52.451) (end 39.796601 51.262399) (width 0.25) (layer F.Cu) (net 3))
 (segment (start 39.796601 51.262399) (end 39.796601 48.559601) (width 0.25) (layer F.Cu) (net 3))
 (segment (start 39.796601 48.559601) (end 39.471599 48.234599) (width 0.25) (layer F.Cu) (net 3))
 (segment (start 39.471599 48.234599) (end 38.608 47.371) (width 0.25) (layer F.Cu) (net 3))
 (segment (start 41.72501 48.166008) (end 41.72501 43.942) (width 0.25) (layer B.Cu) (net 3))
 (segment (start 41.550018 48.341) (end 41.72501 48.166008) (width 0.25) (layer B.Cu) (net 3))
 (segment (start 43.858893 57.001984) (end 41.550018 54.693109) (width 0.25) (layer B.Cu) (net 3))
 (segment (start 53.551516 57.001984) (end 43.858893 57.001984) (width 0.25) (layer B.Cu) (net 3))
 (segment (start 58.3565 52.197) (end 53.551516 57.001984) (width 0.25) (layer B.Cu) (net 3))
 (segment (start 41.550018 54.693109) (end 41.550018 48.341) (width 0.25) (layer B.Cu) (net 3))
 (segment (start 40.513 22.034498) (end 41.742516 23.264014) (width 0.25) (layer F.Cu) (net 5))
 (segment (start 41.802996 24.112502) (end 41.802996 23.28654) (width 0.25) (layer B.Cu) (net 5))
 (segment (start 41.802996 23.28654) (end 41.825522 23.264014) (width 0.25) (layer B.Cu) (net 5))
 (segment (start 41.977987 36.428811) (end 41.977987 24.287493) (width 0.25) (layer B.Cu) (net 5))
 (segment (start 42.17502 36.625844) (end 41.977987 36.428811) (width 0.25) (layer B.Cu) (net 5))
 (segment (start 41.977987 24.287493) (end 41.802996 24.112502) (width 0.25) (layer B.Cu) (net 5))
 (via (at 41.825522 23.264014) (size 0.6) (drill 0.4) (layers F.Cu B.Cu) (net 5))
 (segment (start 41.742516 23.264014) (end 41.825522 23.264014) (width 0.25) (layer F.Cu) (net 5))
 (segment (start 40.513 21.356234) (end 40.513 21.610234) (width 0.25) (layer B.Cu) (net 5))
 (segment (start 40.513 21.610234) (end 40.513 22.034498) (width 0.25) (layer B.Cu) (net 5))
 (segment (start 26.5755 21.1475) (end 27.750501 19.972499) (width 0.25) (layer B.Cu) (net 5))
 (segment (start 39.129265 19.972499) (end 40.513 21.356234) (width 0.25) (layer B.Cu) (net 5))
 (segment (start 27.750501 19.972499) (end 39.129265 19.972499) (width 0.25) (layer B.Cu) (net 5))
 (via (at 40.513 22.034498) (size 0.6) (drill 0.4) (layers F.Cu B.Cu) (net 5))
 (segment (start 44.577 37.2745) (end 44.879001 36.972499) (width 0.25) (layer B.Cu) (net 5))
 (segment (start 44.879001 36.972499) (end 54.488499 36.972499) (width 0.25) (layer B.Cu) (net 5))
 (segment (start 54.488499 36.972499) (end 54.813501 37.297501) (width 0.25) (layer B.Cu) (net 5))
 (segment (start 54.813501 37.297501) (end 55.6635 38.1475) (width 0.25) (layer B.Cu) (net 5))
 (segment (start 42.17502 36.625844) (end 43.928344 36.625844) (width 0.25) (layer F.Cu) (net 5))
 (segment (start 43.928344 36.625844) (end 44.577 37.2745) (width 0.25) (layer F.Cu) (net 5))
 (via (at 44.577 37.2745) (size 0.6) (drill 0.4) (layers F.Cu B.Cu) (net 5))
 (via (at 42.17502 36.625844) (size 0.6) (drill 0.4) (layers F.Cu B.Cu) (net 5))
 (segment (start 42.350011 48.041745) (end 42.350011 38.688999) (width 0.25) (layer B.Cu) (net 5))
 (segment (start 42.17502 48.641) (end 42.17502 48.216736) (width 0.25) (layer B.Cu) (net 5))
 (segment (start 42.17502 48.216736) (end 42.350011 48.041745) (width 0.25) (layer B.Cu) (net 5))
 (segment (start 42.350011 38.688999) (end 42.175019 38.514005) (width 0.25) (layer B.Cu) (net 5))
 (segment (start 42.175019 38.514005) (end 42.17502 36.625844) (width 0.25) (layer B.Cu) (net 5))
 (segment (start 40.4495 48.641) (end 37.338 48.641) (width 0.25) (layer B.Cu) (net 5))
 (segment (start 37.338 48.641) (end 36.068 47.371) (width 0.25) (layer B.Cu) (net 5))
 (segment (start 42.17502 48.641) (end 40.4495 48.641) (width 0.25) (layer F.Cu) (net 5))
 (via (at 40.4495 48.641) (size 0.6) (drill 0.4) (layers F.Cu B.Cu) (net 5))
 (segment (start 42.17502 49.289656) (end 42.17502 48.641) (width 0.25) (layer B.Cu) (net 5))
 (via (at 42.17502 48.641) (size 0.6) (drill 0.4) (layers F.Cu B.Cu) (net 5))
 (segment (start 42.000029 49.464647) (end 42.17502 49.289656) (width 0.25) (layer B.Cu) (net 5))
 (segment (start 42.000029 54.506709) (end 42.000029 49.464647) (width 0.25) (layer B.Cu) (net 5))
 (segment (start 58.3565 49.657) (end 51.461527 56.551973) (width 0.25) (layer B.Cu) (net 5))
 (segment (start 44.045293 56.551973) (end 42.000029 54.506709) (width 0.25) (layer B.Cu) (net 5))
 (segment (start 51.461527 56.551973) (end 44.045293 56.551973) (width 0.25) (layer B.Cu) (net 5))
 (segment (start 43.250031 54.149991) (end 42.116009 54.149991) (width 0.25) (layer F.Cu) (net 6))
 (segment (start 42.116009 54.149991) (end 40.767 55.499) (width 0.25) (layer F.Cu) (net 6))
 (via (at 43.250031 54.149991) (size 0.6) (drill 0.4) (layers F.Cu B.Cu) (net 6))
 (segment (start 43.352999 22.397999) (end 43.053 22.098) (width 0.25) (layer B.Cu) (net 6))
 (segment (start 43.352999 23.412999) (end 43.352999 22.397999) (width 0.25) (layer B.Cu) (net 6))
 (segment (start 43.07504 23.690958) (end 43.352999 23.412999) (width 0.25) (layer B.Cu) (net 6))
 (segment (start 43.07504 25.16804) (end 43.07504 23.690958) (width 0.25) (layer B.Cu) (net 6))
 (segment (start 41.356003 20.401001) (end 41.656002 20.701) (width 0.25) (layer B.Cu) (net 6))
 (segment (start 24.5755 21.1475) (end 26.200512 19.522488) (width 0.25) (layer B.Cu) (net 6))
 (segment (start 42.037 21.082) (end 41.737001 20.781999) (width 0.25) (layer F.Cu) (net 6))
 (via (at 41.656002 20.701) (size 0.6) (drill 0.4) (layers F.Cu B.Cu) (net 6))
 (segment (start 43.053 22.098) (end 42.037 21.082) (width 0.25) (layer F.Cu) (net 6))
 (segment (start 26.200512 19.522488) (end 40.47749 19.522488) (width 0.25) (layer B.Cu) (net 6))
 (segment (start 40.47749 19.522488) (end 41.356003 20.401001) (width 0.25) (layer B.Cu) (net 6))
 (segment (start 41.737001 20.781999) (end 41.656002 20.701) (width 0.25) (layer F.Cu) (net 6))
 (via (at 43.053 22.098) (size 0.6) (drill 0.4) (layers F.Cu B.Cu) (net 6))
 (segment (start 43.07504 34.8615) (end 43.07504 25.16804) (width 0.25) (layer B.Cu) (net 6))
 (segment (start 43.07504 25.16804) (end 43.053 25.146) (width 0.25) (layer B.Cu) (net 6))
 (segment (start 44.6405 34.8615) (end 44.940499 35.161499) (width 0.25) (layer B.Cu) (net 6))
 (segment (start 57.353501 37.297501) (end 58.2035 38.1475) (width 0.25) (layer B.Cu) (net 6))
 (segment (start 44.940499 35.161499) (end 55.217499 35.161499) (width 0.25) (layer B.Cu) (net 6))
 (segment (start 55.217499 35.161499) (end 57.353501 37.297501) (width 0.25) (layer B.Cu) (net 6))
 (segment (start 43.07504 34.8615) (end 44.6405 34.8615) (width 0.25) (layer F.Cu) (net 6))
 (via (at 44.6405 34.8615) (size 0.6) (drill 0.4) (layers F.Cu B.Cu) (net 6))
 (via (at 43.07504 34.8615) (size 0.6) (drill 0.4) (layers F.Cu B.Cu) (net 6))
 (segment (start 43.07504 35.374958) (end 43.07504 34.8615) (width 0.25) (layer B.Cu) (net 6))
 (segment (start 43.250033 49.487465) (end 43.250033 36.139445) (width 0.25) (layer B.Cu) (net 6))
 (segment (start 42.935999 35.513999) (end 43.07504 35.374958) (width 0.25) (layer B.Cu) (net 6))
 (segment (start 42.935999 35.825411) (end 42.935999 35.513999) (width 0.25) (layer B.Cu) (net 6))
 (segment (start 43.250033 36.139445) (end 42.935999 35.825411) (width 0.25) (layer B.Cu) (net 6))
 (segment (start 42.935999 49.801499) (end 43.250033 49.487465) (width 0.25) (layer B.Cu) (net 6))
 (segment (start 42.935999 50.401501) (end 42.935999 49.801499) (width 0.25) (layer B.Cu) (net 6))
 (segment (start 43.07504 50.540542) (end 42.935999 50.401501) (width 0.25) (layer B.Cu) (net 6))
 (segment (start 43.075041 50.960009) (end 43.07504 50.540542) (width 0.25) (layer B.Cu) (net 6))
 (segment (start 44.577 55.47696) (end 43.250031 54.149991) (width 0.25) (layer B.Cu) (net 6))
 (segment (start 43.250031 51.134999) (end 43.075041 50.960009) (width 0.25) (layer B.Cu) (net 6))
 (segment (start 43.250031 54.149991) (end 43.250031 51.134999) (width 0.25) (layer B.Cu) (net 6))
 (segment (start 40.767 55.499) (end 39.116 55.499) (width 0.25) (layer B.Cu) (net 6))
 (segment (start 39.116 55.499) (end 38.608 54.991) (width 0.25) (layer B.Cu) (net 6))
 (via (at 40.767 55.499) (size 0.6) (drill 0.4) (layers F.Cu B.Cu) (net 6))
 (segment (start 40.78904 55.47696) (end 40.767 55.499) (width 0.25) (layer F.Cu) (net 6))
 (segment (start 58.3565 47.117) (end 49.99654 55.47696) (width 0.25) (layer B.Cu) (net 6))
 (segment (start 44.7675 55.47696) (end 44.577 55.47696) (width 0.25) (layer B.Cu) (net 6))
 (segment (start 49.99654 55.47696) (end 44.7675 55.47696) (width 0.25) (layer B.Cu) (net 6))
 (segment (start 43.981931 35.387445) (end 43.981931 32.589069) (width 0.25) (layer B.Cu) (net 1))
 (segment (start 43.981931 32.589069) (end 53.1235 23.4475) (width 0.25) (layer B.Cu) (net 1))
 (segment (start 43.981931 35.387445) (end 43.681932 35.687444) (width 0.25) (layer B.Cu) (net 1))
 (segment (start 43.860999 35.866511) (end 43.681932 35.687444) (width 0.25) (layer B.Cu) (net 1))
 (segment (start 43.555376 35.814) (end 43.681932 35.687444) (width 0.25) (layer F.Cu) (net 1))
 (segment (start 40.4495 35.814) (end 43.555376 35.814) (width 0.25) (layer F.Cu) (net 1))
 (segment (start 43.561 50.1015) (end 43.860999 49.801501) (width 0.25) (layer B.Cu) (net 1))
 (segment (start 43.860999 49.801501) (end 43.860999 35.866511) (width 0.25) (layer B.Cu) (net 1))
 (via (at 43.681932 35.687444) (size 0.6) (drill 0.4) (layers F.Cu B.Cu) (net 1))
 (segment (start 40.4495 35.814) (end 37.87841 35.814) (width 0.25) (layer B.Cu) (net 1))
 (segment (start 37.87841 35.814) (end 37.586899 35.522489) (width 0.25) (layer B.Cu) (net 1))
 (segment (start 37.586899 35.522489) (end 26.200511 35.522489) (width 0.25) (layer B.Cu) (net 1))
 (segment (start 26.200511 35.522489) (end 25.425499 36.297501) (width 0.25) (layer B.Cu) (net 1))
 (segment (start 25.425499 36.297501) (end 24.5755 37.1475) (width 0.25) (layer B.Cu) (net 1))
 (via (at 40.4495 35.814) (size 0.6) (drill 0.4) (layers F.Cu B.Cu) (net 1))
 (segment (start 40.4495 50.1015) (end 38.7985 50.1015) (width 0.25) (layer B.Cu) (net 1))
 (segment (start 38.7985 50.1015) (end 38.608 49.911) (width 0.25) (layer B.Cu) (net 1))
 (segment (start 43.561 50.1015) (end 40.4495 50.1015) (width 0.25) (layer F.Cu) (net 1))
 (via (at 40.4495 50.1015) (size 0.6) (drill 0.4) (layers F.Cu B.Cu) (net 1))
 (via (at 43.561 50.1015) (size 0.6) (drill 0.4) (layers F.Cu B.Cu) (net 1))
 (segment (start 43.561 50.809557) (end 43.561 50.1015) (width 0.25) (layer B.Cu) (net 1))
 (segment (start 43.700042 51.921401) (end 43.700042 50.948599) (width 0.25) (layer B.Cu) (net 1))
 (segment (start 46.706141 54.9275) (end 43.700042 51.921401) (width 0.25) (layer B.Cu) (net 1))
 (segment (start 46.8924 54.9275) (end 46.706141 54.9275) (width 0.25) (layer B.Cu) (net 1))
 (segment (start 58.3565 44.577) (end 57.2429 44.577) (width 0.25) (layer B.Cu) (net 1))
 (segment (start 43.700042 50.948599) (end 43.561 50.809557) (width 0.25) (layer B.Cu) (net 1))
 (segment (start 57.2429 44.577) (end 46.8924 54.9275) (width 0.25) (layer B.Cu) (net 1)))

